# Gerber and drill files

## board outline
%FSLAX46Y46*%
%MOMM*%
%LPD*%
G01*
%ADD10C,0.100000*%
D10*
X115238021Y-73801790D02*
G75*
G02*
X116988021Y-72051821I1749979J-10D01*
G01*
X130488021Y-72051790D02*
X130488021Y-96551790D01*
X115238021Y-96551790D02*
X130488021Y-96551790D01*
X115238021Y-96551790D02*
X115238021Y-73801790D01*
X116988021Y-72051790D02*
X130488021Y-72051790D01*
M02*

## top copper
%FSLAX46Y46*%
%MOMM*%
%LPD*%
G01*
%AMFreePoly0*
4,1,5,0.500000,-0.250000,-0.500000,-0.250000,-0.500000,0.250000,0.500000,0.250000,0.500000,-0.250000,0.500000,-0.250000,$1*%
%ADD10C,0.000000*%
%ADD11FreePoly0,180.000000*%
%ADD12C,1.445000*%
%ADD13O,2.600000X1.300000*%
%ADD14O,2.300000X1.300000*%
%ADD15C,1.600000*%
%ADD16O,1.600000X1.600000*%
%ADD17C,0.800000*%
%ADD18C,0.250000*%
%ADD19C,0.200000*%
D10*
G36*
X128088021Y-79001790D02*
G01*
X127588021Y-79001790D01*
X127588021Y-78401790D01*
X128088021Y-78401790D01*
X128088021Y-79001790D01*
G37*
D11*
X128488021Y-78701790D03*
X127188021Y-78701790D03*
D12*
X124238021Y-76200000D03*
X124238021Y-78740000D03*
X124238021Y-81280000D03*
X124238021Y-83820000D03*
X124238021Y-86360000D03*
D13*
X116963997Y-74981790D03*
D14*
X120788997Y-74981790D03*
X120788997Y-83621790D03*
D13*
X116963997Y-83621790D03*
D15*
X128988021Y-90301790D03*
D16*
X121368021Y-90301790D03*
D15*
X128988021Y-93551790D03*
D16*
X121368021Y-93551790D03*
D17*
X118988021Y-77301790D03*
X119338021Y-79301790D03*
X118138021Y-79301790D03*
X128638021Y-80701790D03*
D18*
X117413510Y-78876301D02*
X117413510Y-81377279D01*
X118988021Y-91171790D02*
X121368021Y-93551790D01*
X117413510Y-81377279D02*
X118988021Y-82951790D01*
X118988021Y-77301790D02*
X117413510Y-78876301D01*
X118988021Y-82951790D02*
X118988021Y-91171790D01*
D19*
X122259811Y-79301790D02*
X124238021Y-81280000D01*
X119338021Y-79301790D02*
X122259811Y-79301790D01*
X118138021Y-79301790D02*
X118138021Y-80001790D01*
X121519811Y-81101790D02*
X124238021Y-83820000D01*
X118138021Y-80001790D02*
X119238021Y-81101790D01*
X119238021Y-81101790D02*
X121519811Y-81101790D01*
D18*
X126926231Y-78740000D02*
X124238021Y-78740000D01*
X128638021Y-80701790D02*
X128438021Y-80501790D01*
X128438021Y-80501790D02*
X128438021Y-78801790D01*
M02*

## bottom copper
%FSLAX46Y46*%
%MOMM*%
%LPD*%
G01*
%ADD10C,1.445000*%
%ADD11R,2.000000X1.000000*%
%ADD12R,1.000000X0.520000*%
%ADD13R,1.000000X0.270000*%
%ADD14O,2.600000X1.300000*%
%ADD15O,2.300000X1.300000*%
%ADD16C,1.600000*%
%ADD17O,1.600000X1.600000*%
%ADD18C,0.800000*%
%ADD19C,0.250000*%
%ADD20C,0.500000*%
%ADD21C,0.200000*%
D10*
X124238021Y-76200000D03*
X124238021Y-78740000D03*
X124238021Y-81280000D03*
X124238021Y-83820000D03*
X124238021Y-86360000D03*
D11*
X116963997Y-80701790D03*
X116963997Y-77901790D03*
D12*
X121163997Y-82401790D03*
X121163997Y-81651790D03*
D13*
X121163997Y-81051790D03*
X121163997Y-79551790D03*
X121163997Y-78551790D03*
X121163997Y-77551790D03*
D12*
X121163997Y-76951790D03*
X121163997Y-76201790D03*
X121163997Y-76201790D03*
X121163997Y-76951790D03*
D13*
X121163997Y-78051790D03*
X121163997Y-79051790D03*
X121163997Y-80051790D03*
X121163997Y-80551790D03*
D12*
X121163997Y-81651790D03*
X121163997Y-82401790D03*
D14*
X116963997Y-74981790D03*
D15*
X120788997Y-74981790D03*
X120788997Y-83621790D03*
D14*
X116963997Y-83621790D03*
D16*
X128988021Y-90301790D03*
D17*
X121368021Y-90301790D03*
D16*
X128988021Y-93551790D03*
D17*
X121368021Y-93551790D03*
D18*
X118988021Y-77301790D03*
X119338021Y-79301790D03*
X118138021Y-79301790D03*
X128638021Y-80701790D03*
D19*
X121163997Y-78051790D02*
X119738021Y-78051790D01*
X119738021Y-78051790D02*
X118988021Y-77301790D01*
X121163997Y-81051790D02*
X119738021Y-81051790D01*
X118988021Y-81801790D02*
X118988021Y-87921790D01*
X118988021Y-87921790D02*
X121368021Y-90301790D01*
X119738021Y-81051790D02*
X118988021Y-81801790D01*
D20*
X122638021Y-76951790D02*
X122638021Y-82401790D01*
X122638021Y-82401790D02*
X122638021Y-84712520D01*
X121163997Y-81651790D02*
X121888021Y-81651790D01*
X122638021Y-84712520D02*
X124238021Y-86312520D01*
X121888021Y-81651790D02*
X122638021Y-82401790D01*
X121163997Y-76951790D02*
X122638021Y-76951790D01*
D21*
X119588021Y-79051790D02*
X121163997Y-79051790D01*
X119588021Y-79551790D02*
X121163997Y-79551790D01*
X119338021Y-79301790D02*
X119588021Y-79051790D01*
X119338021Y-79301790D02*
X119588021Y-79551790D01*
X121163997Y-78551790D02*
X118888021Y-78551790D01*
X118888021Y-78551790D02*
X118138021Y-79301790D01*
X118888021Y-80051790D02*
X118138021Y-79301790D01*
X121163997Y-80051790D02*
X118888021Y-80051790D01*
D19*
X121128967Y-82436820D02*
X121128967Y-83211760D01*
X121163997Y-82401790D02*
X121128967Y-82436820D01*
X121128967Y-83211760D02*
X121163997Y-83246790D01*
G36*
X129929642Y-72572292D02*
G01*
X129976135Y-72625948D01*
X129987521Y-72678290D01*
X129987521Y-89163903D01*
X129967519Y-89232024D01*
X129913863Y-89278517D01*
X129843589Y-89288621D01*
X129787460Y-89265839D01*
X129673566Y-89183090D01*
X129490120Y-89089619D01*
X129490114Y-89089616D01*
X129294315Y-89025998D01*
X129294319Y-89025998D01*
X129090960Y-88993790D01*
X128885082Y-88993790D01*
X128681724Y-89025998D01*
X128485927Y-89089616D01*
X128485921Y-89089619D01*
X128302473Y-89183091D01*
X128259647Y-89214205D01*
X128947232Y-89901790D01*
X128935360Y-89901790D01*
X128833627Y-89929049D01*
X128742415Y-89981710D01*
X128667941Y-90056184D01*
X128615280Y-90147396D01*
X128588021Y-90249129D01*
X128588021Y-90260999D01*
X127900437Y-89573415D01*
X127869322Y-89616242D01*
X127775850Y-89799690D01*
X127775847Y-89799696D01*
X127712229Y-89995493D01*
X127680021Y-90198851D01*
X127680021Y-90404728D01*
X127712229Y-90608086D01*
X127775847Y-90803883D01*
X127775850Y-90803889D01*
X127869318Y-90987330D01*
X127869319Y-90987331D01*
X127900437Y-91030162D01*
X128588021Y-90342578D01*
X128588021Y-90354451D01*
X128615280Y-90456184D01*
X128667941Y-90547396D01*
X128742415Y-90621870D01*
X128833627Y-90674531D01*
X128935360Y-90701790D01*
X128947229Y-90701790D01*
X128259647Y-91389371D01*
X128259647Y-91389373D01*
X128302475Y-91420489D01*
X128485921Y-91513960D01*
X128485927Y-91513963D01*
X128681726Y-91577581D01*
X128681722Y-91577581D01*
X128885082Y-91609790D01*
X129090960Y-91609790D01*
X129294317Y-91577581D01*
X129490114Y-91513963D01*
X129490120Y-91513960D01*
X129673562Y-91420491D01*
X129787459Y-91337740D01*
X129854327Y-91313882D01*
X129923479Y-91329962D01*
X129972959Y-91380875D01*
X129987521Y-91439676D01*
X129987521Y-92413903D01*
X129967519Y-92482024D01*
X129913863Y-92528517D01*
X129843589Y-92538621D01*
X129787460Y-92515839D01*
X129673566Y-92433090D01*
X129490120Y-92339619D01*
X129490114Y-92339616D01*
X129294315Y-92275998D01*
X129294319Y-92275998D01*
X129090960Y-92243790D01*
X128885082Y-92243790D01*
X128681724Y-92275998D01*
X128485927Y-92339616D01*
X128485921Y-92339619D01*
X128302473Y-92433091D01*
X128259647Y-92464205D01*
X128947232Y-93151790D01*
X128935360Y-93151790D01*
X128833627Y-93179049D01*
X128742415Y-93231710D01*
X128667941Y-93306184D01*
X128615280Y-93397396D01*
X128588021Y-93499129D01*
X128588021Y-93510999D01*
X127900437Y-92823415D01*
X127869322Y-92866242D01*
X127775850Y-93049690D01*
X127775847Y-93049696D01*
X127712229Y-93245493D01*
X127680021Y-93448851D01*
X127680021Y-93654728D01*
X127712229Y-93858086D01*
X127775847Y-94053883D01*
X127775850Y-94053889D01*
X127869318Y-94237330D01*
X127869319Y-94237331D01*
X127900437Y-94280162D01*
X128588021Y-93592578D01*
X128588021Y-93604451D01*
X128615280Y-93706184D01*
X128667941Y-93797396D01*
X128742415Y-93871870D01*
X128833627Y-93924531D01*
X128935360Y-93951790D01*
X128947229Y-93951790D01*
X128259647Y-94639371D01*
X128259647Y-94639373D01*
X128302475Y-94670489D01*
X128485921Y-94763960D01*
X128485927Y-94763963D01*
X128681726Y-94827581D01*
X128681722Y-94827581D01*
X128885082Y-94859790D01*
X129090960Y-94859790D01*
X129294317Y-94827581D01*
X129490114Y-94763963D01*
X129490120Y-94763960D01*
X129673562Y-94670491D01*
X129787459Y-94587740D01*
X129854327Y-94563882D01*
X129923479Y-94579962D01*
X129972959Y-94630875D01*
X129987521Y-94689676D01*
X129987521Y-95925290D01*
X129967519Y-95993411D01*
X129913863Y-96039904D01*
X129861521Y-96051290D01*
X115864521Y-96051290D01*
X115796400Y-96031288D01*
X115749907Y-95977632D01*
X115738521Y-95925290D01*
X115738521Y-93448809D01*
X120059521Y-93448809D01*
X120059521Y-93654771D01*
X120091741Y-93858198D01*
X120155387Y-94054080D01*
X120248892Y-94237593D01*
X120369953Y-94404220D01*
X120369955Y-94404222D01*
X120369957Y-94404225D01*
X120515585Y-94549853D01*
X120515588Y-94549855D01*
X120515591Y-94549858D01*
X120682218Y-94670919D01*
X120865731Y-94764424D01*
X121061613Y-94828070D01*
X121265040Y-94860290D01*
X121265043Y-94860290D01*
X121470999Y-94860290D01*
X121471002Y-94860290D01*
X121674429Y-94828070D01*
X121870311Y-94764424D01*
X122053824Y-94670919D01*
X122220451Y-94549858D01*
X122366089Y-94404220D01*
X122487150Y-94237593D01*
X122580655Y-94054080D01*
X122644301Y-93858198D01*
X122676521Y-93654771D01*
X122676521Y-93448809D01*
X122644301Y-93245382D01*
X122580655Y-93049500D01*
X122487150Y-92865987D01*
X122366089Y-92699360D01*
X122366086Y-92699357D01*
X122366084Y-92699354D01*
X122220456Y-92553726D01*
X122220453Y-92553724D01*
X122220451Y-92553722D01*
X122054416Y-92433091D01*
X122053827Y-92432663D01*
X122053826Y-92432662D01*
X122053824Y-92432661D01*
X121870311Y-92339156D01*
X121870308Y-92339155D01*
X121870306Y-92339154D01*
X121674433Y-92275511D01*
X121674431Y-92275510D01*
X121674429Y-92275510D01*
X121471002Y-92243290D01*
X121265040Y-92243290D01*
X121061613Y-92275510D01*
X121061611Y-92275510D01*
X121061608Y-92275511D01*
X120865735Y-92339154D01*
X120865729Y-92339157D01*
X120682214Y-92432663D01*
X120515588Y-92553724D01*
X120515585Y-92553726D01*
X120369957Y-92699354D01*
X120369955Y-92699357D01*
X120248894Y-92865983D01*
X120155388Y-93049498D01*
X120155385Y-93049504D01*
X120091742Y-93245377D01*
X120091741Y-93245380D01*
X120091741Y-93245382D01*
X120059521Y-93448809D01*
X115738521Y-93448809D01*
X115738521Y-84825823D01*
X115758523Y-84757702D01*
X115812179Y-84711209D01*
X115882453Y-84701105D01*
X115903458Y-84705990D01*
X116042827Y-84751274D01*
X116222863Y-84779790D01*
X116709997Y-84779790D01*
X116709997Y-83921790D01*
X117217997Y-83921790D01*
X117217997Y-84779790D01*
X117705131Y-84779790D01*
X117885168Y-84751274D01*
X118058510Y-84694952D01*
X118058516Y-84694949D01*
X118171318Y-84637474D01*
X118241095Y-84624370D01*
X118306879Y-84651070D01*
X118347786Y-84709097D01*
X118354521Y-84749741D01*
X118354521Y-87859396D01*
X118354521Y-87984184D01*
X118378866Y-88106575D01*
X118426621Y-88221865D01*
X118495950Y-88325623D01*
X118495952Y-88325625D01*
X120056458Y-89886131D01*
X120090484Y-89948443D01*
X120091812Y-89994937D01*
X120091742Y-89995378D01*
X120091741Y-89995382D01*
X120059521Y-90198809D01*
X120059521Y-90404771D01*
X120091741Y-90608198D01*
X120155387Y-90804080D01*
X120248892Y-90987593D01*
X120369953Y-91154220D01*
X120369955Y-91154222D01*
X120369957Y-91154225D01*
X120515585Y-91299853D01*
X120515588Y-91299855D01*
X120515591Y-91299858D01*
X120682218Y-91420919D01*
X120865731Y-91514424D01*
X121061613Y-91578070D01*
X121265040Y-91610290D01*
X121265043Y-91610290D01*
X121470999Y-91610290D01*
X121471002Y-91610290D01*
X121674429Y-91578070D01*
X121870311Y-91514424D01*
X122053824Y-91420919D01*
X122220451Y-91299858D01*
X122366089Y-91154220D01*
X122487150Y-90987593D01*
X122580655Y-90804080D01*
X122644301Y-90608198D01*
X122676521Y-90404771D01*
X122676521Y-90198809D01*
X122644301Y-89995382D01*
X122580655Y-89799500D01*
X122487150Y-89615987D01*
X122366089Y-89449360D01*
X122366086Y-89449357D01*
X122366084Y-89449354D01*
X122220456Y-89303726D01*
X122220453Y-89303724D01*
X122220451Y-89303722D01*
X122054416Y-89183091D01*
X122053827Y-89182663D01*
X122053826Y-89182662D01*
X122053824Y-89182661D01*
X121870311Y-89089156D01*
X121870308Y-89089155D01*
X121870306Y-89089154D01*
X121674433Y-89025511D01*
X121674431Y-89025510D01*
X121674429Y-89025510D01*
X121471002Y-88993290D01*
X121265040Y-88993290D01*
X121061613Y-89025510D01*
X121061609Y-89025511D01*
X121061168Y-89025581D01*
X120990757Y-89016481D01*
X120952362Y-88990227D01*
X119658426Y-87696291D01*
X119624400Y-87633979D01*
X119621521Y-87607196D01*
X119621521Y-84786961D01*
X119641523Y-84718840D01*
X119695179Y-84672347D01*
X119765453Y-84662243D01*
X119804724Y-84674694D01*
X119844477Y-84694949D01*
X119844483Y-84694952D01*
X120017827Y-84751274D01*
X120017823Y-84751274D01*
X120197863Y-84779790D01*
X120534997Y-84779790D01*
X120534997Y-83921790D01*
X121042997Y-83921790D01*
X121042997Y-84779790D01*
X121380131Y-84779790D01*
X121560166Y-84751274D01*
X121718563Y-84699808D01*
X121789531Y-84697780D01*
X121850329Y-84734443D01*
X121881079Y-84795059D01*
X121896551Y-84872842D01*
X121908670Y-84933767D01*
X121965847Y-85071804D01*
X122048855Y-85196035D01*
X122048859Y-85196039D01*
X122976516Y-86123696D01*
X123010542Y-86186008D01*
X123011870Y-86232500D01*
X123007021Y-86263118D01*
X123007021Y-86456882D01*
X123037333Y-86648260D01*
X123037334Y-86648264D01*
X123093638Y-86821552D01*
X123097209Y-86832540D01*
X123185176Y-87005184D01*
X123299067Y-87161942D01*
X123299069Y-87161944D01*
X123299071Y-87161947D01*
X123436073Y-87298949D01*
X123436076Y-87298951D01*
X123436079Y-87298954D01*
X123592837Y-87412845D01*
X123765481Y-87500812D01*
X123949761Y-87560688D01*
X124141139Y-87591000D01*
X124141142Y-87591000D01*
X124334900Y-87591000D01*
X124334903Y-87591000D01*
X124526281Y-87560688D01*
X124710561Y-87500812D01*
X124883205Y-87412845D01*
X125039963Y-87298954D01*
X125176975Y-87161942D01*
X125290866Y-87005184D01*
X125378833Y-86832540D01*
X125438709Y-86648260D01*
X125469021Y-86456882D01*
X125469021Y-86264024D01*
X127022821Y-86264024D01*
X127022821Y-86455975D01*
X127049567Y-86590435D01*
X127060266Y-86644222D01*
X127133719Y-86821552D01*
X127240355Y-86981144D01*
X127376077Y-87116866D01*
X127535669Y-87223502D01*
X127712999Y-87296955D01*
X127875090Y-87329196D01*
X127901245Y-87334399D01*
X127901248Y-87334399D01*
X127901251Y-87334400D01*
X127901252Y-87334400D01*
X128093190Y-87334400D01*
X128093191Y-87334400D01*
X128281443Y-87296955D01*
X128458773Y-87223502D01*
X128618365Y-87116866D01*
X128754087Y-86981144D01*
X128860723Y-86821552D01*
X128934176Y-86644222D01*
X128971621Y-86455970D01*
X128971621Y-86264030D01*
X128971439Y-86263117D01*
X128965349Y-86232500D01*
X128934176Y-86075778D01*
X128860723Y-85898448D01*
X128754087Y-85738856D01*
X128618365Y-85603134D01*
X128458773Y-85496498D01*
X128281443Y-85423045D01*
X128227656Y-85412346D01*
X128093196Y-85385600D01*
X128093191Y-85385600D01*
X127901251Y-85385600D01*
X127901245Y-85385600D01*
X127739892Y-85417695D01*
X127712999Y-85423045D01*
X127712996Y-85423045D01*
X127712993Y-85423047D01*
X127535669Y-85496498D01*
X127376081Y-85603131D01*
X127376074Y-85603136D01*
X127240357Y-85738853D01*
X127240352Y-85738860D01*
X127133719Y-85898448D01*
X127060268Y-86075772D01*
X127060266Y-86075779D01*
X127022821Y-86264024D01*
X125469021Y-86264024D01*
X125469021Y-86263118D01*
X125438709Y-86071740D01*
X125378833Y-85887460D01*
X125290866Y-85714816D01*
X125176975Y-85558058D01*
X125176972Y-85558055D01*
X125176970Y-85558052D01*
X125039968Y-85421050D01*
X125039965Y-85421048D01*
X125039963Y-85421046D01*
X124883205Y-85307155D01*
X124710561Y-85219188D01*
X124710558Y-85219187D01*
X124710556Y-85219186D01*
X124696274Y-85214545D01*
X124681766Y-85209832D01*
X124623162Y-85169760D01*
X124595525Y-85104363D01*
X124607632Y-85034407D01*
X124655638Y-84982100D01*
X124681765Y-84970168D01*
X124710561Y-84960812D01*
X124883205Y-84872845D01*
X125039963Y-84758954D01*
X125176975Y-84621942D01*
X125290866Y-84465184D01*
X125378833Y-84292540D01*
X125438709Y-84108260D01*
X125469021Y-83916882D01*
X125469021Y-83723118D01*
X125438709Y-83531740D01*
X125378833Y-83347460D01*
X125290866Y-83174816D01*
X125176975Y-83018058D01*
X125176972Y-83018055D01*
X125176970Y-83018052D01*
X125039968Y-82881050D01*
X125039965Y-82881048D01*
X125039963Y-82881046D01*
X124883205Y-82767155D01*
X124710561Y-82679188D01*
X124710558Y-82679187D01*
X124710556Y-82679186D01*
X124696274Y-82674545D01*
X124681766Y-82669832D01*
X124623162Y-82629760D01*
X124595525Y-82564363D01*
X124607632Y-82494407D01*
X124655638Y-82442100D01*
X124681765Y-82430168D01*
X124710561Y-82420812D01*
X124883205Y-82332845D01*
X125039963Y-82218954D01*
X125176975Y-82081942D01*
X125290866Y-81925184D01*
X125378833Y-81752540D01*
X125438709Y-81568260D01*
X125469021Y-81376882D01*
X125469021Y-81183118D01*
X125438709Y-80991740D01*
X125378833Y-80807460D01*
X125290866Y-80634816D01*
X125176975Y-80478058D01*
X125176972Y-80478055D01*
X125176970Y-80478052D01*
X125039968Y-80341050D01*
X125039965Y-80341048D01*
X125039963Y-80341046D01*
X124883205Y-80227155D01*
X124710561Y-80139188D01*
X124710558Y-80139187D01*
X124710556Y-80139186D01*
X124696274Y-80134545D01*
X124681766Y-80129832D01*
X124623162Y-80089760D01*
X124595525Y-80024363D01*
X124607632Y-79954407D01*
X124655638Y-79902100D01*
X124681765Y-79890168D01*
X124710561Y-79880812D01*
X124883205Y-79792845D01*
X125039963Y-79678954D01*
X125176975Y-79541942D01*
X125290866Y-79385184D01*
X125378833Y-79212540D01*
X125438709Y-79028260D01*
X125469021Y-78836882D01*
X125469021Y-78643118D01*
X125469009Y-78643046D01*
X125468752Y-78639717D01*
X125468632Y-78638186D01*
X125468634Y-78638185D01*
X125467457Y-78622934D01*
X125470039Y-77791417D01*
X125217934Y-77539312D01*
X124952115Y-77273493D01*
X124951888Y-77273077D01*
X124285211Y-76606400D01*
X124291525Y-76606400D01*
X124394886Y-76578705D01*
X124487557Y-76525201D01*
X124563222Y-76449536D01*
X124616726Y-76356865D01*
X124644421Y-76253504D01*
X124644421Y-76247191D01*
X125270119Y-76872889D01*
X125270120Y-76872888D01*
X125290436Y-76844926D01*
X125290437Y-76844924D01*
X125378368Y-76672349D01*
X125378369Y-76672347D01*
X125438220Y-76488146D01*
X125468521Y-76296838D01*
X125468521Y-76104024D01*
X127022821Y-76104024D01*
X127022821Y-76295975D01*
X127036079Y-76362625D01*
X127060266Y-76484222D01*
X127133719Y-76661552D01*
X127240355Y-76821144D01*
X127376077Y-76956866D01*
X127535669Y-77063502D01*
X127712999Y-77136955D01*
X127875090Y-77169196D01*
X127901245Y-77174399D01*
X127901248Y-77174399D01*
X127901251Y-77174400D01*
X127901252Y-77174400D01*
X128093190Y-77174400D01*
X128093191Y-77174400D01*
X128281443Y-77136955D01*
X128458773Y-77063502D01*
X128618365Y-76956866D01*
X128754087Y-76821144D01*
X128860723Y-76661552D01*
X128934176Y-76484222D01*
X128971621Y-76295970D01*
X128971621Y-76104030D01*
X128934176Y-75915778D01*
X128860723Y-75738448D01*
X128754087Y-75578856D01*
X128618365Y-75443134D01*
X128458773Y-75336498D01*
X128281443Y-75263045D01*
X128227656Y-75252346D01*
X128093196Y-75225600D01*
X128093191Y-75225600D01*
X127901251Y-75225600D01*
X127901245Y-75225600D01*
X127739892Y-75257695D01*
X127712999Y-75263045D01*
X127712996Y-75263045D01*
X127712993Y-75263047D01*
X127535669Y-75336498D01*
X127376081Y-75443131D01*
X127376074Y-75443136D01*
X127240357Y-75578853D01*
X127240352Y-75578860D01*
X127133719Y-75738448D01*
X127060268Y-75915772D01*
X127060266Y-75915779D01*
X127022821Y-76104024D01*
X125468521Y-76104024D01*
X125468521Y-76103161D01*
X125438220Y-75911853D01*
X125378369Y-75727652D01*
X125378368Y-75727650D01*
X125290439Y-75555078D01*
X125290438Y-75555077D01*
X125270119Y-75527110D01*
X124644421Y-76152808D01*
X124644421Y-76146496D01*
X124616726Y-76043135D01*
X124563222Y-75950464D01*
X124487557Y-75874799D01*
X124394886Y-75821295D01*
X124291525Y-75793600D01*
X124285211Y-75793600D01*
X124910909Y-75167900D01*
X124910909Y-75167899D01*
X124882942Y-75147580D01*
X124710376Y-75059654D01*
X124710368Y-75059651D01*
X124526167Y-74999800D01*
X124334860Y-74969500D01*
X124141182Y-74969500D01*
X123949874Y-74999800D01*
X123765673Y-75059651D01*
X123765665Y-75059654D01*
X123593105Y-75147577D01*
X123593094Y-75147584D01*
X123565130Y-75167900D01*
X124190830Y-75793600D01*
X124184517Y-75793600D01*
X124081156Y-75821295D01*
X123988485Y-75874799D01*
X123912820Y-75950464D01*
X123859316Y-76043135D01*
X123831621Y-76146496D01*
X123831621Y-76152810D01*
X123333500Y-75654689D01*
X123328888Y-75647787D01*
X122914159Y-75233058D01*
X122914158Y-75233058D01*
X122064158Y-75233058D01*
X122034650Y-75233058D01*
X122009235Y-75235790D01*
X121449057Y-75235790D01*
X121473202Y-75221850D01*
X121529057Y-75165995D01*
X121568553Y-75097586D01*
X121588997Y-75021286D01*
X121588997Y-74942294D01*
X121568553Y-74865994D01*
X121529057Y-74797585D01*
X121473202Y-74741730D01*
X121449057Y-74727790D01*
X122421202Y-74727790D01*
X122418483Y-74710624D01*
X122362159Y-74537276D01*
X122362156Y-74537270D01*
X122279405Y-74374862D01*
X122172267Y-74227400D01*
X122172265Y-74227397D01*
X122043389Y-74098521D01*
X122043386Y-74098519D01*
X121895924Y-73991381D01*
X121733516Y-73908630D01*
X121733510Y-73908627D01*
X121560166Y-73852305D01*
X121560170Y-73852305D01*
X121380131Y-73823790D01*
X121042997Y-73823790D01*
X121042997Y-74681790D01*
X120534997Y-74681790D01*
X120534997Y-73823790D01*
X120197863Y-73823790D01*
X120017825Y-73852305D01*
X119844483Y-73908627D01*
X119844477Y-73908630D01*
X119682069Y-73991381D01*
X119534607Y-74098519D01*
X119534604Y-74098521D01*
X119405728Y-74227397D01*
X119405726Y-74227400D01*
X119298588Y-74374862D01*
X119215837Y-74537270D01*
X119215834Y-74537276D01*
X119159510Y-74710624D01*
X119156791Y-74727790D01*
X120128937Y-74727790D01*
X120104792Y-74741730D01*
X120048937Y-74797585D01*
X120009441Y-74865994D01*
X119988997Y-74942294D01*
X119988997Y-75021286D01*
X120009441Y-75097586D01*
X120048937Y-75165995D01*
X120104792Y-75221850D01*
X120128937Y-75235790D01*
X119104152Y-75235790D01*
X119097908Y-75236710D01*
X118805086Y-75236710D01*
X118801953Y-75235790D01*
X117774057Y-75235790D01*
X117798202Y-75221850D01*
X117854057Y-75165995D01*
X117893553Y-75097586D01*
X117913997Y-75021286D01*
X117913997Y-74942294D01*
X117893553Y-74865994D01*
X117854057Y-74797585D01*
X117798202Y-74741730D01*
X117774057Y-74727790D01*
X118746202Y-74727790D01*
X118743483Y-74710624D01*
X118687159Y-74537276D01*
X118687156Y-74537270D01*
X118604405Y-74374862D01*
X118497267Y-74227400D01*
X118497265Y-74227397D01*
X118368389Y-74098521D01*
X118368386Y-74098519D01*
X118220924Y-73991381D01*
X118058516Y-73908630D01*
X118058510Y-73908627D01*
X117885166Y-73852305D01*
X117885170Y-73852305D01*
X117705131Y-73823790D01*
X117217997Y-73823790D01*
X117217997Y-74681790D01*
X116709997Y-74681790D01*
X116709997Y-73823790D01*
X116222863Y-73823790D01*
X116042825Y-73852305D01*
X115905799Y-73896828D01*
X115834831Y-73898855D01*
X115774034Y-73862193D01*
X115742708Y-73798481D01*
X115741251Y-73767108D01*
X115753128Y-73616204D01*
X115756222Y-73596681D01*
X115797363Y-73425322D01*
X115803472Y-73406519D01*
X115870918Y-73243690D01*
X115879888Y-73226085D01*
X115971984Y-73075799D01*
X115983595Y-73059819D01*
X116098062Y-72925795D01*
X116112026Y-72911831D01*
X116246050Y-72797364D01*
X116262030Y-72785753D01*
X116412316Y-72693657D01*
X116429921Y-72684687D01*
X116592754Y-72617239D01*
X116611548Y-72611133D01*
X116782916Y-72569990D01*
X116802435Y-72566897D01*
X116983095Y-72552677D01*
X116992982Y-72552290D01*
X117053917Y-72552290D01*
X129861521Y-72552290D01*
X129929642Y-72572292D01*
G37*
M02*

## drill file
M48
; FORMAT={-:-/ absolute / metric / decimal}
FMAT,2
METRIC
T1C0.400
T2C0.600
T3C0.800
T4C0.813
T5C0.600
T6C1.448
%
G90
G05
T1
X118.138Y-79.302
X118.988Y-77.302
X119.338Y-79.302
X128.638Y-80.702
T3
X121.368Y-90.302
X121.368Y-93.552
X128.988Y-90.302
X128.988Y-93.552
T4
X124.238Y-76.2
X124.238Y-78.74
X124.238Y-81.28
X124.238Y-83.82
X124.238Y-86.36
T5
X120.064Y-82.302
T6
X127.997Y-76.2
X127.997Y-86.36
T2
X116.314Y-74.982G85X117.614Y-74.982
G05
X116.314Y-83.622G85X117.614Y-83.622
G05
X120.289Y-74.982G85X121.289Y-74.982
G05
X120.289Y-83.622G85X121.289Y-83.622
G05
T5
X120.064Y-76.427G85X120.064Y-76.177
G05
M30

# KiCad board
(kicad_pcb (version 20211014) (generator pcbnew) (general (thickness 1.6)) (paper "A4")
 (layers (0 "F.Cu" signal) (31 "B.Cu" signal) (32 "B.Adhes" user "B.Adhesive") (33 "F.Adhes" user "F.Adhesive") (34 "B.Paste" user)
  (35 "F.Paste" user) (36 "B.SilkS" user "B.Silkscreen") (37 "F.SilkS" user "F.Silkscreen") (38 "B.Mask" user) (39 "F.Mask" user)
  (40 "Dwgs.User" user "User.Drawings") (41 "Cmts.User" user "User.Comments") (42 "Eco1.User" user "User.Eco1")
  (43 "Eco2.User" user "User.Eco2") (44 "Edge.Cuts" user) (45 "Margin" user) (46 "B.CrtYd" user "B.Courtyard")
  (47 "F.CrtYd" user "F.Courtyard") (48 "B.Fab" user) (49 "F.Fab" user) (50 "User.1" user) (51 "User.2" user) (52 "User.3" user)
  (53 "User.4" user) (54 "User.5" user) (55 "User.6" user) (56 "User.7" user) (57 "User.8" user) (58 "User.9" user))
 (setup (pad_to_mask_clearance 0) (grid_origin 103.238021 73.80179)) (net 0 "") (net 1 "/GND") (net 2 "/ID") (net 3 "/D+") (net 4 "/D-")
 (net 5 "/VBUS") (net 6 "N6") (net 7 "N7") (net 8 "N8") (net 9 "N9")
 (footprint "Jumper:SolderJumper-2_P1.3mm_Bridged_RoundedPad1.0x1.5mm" (layer "F.Cu") (at 127.838021 78.70179 180)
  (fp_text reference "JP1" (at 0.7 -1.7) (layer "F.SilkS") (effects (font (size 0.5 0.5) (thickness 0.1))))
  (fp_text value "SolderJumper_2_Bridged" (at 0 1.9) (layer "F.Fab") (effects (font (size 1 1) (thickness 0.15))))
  (fp_poly (pts (xy 0.25 -0.3) (xy -0.25 -0.3) (xy -0.25 0.3) (xy 0.25 0.3)) (layer "F.Cu") (width 0) (fill solid))
  (pad "1" smd custom (at -0.65 0 180) (size 1 0.5) (layers "F.Cu" "F.Mask") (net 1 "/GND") (zone_connect 2)
   (options (clearance outline) (anchor rect)) (primitives))
  (pad "2" smd custom (at 0.65 0 180) (size 1 0.5) (layers "F.Cu" "F.Mask") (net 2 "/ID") (zone_connect 2)
   (options (clearance outline) (anchor rect)) (primitives)))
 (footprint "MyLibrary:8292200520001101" (layer "F.Cu") (at 124.238021 76.2)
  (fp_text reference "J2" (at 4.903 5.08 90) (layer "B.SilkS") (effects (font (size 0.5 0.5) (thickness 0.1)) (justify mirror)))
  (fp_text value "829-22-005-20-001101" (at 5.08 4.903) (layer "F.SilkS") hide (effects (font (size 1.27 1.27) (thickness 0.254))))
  (pad "" np_thru_hole circle (at 3.7592 10.16 90) (size 1.4478 1.4478) (drill 1.4478) (layers F&B.Cu *.Mask))
  (pad "" np_thru_hole circle (at 3.7592 0 90) (size 1.4478 1.4478) (drill 1.4478) (layers F&B.Cu *.Mask))
  (pad "1" thru_hole circle (at 0 0 90) (size 1.445 1.445) (drill 0.8128) (layers *.Cu *.Mask) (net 1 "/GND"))
  (pad "2" thru_hole circle (at 0 2.54 90) (size 1.445 1.445) (drill 0.8128) (layers *.Cu *.Mask) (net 2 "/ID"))
  (pad "3" thru_hole circle (at 0 5.08 90) (size 1.445 1.445) (drill 0.8128) (layers *.Cu *.Mask) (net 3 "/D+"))
  (pad "4" thru_hole circle (at 0 7.62 90) (size 1.445 1.445) (drill 0.8128) (layers *.Cu *.Mask) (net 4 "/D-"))
  (pad "5" thru_hole circle (at 0 10.16 90) (size 1.445 1.445) (drill 0.8128) (layers *.Cu *.Mask) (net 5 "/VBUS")))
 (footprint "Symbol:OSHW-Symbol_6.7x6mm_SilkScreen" (layer "F.Cu") (at 118.488021 79.30179 90)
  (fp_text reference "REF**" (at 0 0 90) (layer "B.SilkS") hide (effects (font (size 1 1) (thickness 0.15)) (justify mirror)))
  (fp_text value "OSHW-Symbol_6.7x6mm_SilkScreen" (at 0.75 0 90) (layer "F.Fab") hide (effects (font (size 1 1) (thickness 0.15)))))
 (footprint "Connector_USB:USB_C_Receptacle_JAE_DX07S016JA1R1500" (layer "B.Cu") (at 118.113997 79.30179 90)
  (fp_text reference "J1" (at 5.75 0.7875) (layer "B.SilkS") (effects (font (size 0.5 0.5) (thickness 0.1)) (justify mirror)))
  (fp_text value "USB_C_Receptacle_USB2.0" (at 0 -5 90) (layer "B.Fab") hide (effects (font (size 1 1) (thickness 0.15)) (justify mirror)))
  (pad "" smd rect (at -1.4 -1.15 90) (size 1 2) (layers "B.Cu" "B.Paste" "B.Mask"))
  (pad "" np_thru_hole circle (at -3 1.95 90) (size 0.6 0.6) (drill 0.6) (layers F&B.Cu *.Mask))
  (pad "" np_thru_hole oval (at 3 1.95 90) (size 0.85 0.6) (drill oval 0.85 0.6) (layers F&B.Cu *.Mask))
  (pad "" smd rect (at 1.4 -1.15 90) (size 1 2) (layers "B.Cu" "B.Paste" "B.Mask"))
  (pad "A1" smd rect (at -3.1 3.05 90) (size 0.52 1) (layers "B.Cu" "B.Paste" "B.Mask") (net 1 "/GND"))
  (pad "A4" smd rect (at -2.35 3.05 90) (size 0.52 1) (layers "B.Cu" "B.Paste" "B.Mask") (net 5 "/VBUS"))
  (pad "A5" smd rect (at -1.75 3.05 90) (size 0.27 1) (layers "B.Cu" "B.Paste" "B.Mask") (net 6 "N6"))
  (pad "A6" smd rect (at -0.25 3.05 90) (size 0.27 1) (layers "B.Cu" "B.Paste" "B.Mask") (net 3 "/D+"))
  (pad "A7" smd rect (at 0.75 3.05 90) (size 0.27 1) (layers "B.Cu" "B.Paste" "B.Mask") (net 4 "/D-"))
  (pad "A8" smd rect (at 1.75 3.05 90) (size 0.27 1) (layers "B.Cu" "B.Paste" "B.Mask") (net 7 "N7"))
  (pad "A9" smd rect (at 2.35 3.05 90) (size 0.52 1) (layers "B.Cu" "B.Paste" "B.Mask") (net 5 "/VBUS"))
  (pad "A12" smd rect (at 3.1 3.05 90) (size 0.52 1) (layers "B.Cu" "B.Paste" "B.Mask") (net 1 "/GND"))
  (pad "B1" smd rect (at 3.1 3.05 90) (size 0.52 1) (layers "B.Cu" "B.Paste" "B.Mask") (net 1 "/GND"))
  (pad "B4" smd rect (at 2.35 3.05 90) (size 0.52 1) (layers "B.Cu" "B.Paste" "B.Mask") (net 5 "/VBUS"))
  (pad "B5" smd rect (at 1.25 3.05 90) (size 0.27 1) (layers "B.Cu" "B.Paste" "B.Mask") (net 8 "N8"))
  (pad "B6" smd rect (at 0.25 3.05 90) (size 0.27 1) (layers "B.Cu" "B.Paste" "B.Mask") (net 3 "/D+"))
  (pad "B7" smd rect (at -0.75 3.05 90) (size 0.27 1) (layers "B.Cu" "B.Paste" "B.Mask") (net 4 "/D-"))
  (pad "B8" smd rect (at -1.25 3.05 90) (size 0.27 1) (layers "B.Cu" "B.Paste" "B.Mask") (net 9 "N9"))
  (pad "B9" smd rect (at -2.35 3.05 90) (size 0.52 1) (layers "B.Cu" "B.Paste" "B.Mask") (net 5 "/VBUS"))
  (pad "B12" smd rect (at -3.1 3.05 90) (size 0.52 1) (layers "B.Cu" "B.Paste" "B.Mask") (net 1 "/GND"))
  (pad "S1" thru_hole oval (at 4.32 -1.15 90) (size 1.3 2.6) (drill oval 0.6 1.9) (layers *.Cu *.Mask) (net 1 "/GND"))
  (pad "S1" thru_hole oval (at 4.32 2.675 90) (size 1.3 2.3) (drill oval 0.6 1.6) (layers *.Cu *.Mask) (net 1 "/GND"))
  (pad "S1" thru_hole oval (at -4.32 2.675 90) (size 1.3 2.3) (drill oval 0.6 1.6) (layers *.Cu *.Mask) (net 1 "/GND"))
  (pad "S1" thru_hole oval (at -4.32 -1.15 90) (size 1.3 2.6) (drill oval 0.6 1.9) (layers *.Cu *.Mask) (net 1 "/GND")))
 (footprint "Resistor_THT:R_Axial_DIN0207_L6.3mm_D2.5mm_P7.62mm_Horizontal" (layer "B.Cu") (at 128.988021 90.30179 180)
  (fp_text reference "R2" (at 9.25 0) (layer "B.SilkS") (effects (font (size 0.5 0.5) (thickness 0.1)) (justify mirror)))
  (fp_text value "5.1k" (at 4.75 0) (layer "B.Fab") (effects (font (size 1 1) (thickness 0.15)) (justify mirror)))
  (pad "1" thru_hole circle (at 0 0 180) (size 1.6 1.6) (drill 0.8) (layers *.Cu *.Mask) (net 1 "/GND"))
  (pad "2" thru_hole oval (at 7.62 0 180) (size 1.6 1.6) (drill 0.8) (layers *.Cu *.Mask) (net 6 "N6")))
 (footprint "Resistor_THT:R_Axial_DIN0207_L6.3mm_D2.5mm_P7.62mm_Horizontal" (layer "B.Cu") (at 128.988021 93.55179 180)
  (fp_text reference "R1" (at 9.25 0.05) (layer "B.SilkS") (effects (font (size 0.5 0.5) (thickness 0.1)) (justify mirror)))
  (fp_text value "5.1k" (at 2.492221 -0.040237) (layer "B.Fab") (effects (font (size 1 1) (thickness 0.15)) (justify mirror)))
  (pad "1" thru_hole circle (at 0 0 180) (size 1.6 1.6) (drill 0.8) (layers *.Cu *.Mask) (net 1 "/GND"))
  (pad "2" thru_hole oval (at 7.62 0 180) (size 1.6 1.6) (drill 0.8) (layers *.Cu *.Mask) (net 8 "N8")))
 (gr_arc (start 115.238021 73.80179) (mid 115.750587 72.564359) (end 116.988021 72.05179) (layer "Edge.Cuts") (width 0.1))
 (gr_line (start 130.488021 72.05179) (end 130.488021 96.55179) (layer "Edge.Cuts") (width 0.1))
 (gr_line (start 115.238021 96.55179) (end 130.488021 96.55179) (layer "Edge.Cuts") (width 0.1))
 (gr_line (start 115.238021 96.55179) (end 115.238021 73.80179) (layer "Edge.Cuts") (width 0.1))
 (gr_line (start 116.988021 72.05179) (end 130.488021 72.05179) (layer "Edge.Cuts") (width 0.1))
 (segment (start 117.41351 78.876301) (end 117.41351 81.377279) (width 0.25) (layer "F.Cu") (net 8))
 (segment (start 118.988021 91.17179) (end 121.368021 93.55179) (width 0.25) (layer "F.Cu") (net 8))
 (segment (start 117.41351 81.377279) (end 118.988021 82.95179) (width 0.25) (layer "F.Cu") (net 8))
 (segment (start 118.988021 77.30179) (end 117.41351 78.876301) (width 0.25) (layer "F.Cu") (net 8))
 (segment (start 118.988021 82.95179) (end 118.988021 91.17179) (width 0.25) (layer "F.Cu") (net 8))
 (via (at 118.988021 77.30179) (size 0.8) (drill 0.4) (layers "F.Cu" "B.Cu") (free) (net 8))
 (segment (start 121.163997 78.05179) (end 119.738021 78.05179) (width 0.25) (layer "B.Cu") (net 8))
 (segment (start 119.738021 78.05179) (end 118.988021 77.30179) (width 0.25) (layer "B.Cu") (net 8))
 (segment (start 121.163997 81.05179) (end 119.738021 81.05179) (width 0.25) (layer "B.Cu") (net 6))
 (segment (start 118.988021 81.80179) (end 118.988021 87.92179) (width 0.25) (layer "B.Cu") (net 6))
 (segment (start 118.988021 87.92179) (end 121.368021 90.30179) (width 0.25) (layer "B.Cu") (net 6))
 (segment (start 119.738021 81.05179) (end 118.988021 81.80179) (width 0.25) (layer "B.Cu") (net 6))
 (segment (start 122.638021 76.95179) (end 122.638021 82.40179) (width 0.5) (layer "B.Cu") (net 5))
 (segment (start 122.638021 82.40179) (end 122.638021 84.71252) (width 0.5) (layer "B.Cu") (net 5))
 (segment (start 121.163997 81.65179) (end 121.888021 81.65179) (width 0.5) (layer "B.Cu") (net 5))
 (segment (start 122.638021 84.71252) (end 124.238021 86.31252) (width 0.5) (layer "B.Cu") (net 5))
 (segment (start 121.888021 81.65179) (end 122.638021 82.40179) (width 0.5) (layer "B.Cu") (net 5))
 (segment (start 121.163997 76.95179) (end 122.638021 76.95179) (width 0.5) (layer "B.Cu") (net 5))
 (segment (start 122.259811 79.30179) (end 124.238021 81.28) (width 0.2) (layer "F.Cu") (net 3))
 (segment (start 119.338021 79.30179) (end 122.259811 79.30179) (width 0.2) (layer "F.Cu") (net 3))
 (via (at 119.338021 79.30179) (size 0.8) (drill 0.4) (layers "F.Cu" "B.Cu") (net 3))
 (segment (start 119.588021 79.05179) (end 121.163997 79.05179) (width 0.2) (layer "B.Cu") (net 3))
 (segment (start 119.588021 79.55179) (end 121.163997 79.55179) (width 0.2) (layer "B.Cu") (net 3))
 (segment (start 119.338021 79.30179) (end 119.588021 79.05179) (width 0.2) (layer "B.Cu") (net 3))
 (segment (start 119.338021 79.30179) (end 119.588021 79.55179) (width 0.2) (layer "B.Cu") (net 3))
 (segment (start 118.138021 79.30179) (end 118.138021 80.00179) (width 0.2) (layer "F.Cu") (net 4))
 (segment (start 121.519811 81.10179) (end 124.238021 83.82) (width 0.2) (layer "F.Cu") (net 4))
 (segment (start 118.138021 80.00179) (end 119.238021 81.10179) (width 0.2) (layer "F.Cu") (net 4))
 (segment (start 119.238021 81.10179) (end 121.519811 81.10179) (width 0.2) (layer "F.Cu") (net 4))
 (via (at 118.138021 79.30179) (size 0.8) (drill 0.4) (layers "F.Cu" "B.Cu") (free) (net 4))
 (segment (start 121.163997 78.55179) (end 118.888021 78.55179) (width 0.2) (layer "B.Cu") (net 4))
 (segment (start 118.888021 78.55179) (end 118.138021 79.30179) (width 0.2) (layer "B.Cu") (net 4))
 (segment (start 118.888021 80.05179) (end 118.138021 79.30179) (width 0.2) (layer "B.Cu") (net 4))
 (segment (start 121.163997 80.05179) (end 118.888021 80.05179) (width 0.2) (layer "B.Cu") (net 4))
 (segment (start 126.926231 78.74) (end 124.238021 78.74) (width 0.25) (layer "F.Cu") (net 2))
 (segment (start 128.638021 80.70179) (end 128.438021 80.50179) (width 0.25) (layer "F.Cu") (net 1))
 (segment (start 128.438021 80.50179) (end 128.438021 78.80179) (width 0.25) (layer "F.Cu") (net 1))
 (via (at 128.638021 80.70179) (size 0.8) (drill 0.4) (layers "F.Cu" "B.Cu") (free) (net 1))
 (segment (start 121.128967 82.43682) (end 121.128967 83.21176) (width 0.25) (layer "B.Cu") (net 1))
 (segment (start 121.163997 82.40179) (end 121.128967 82.43682) (width 0.25) (layer "B.Cu") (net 1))
 (segment (start 121.128967 83.21176) (end 121.163997 83.24679) (width 0.25) (layer "B.Cu") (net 1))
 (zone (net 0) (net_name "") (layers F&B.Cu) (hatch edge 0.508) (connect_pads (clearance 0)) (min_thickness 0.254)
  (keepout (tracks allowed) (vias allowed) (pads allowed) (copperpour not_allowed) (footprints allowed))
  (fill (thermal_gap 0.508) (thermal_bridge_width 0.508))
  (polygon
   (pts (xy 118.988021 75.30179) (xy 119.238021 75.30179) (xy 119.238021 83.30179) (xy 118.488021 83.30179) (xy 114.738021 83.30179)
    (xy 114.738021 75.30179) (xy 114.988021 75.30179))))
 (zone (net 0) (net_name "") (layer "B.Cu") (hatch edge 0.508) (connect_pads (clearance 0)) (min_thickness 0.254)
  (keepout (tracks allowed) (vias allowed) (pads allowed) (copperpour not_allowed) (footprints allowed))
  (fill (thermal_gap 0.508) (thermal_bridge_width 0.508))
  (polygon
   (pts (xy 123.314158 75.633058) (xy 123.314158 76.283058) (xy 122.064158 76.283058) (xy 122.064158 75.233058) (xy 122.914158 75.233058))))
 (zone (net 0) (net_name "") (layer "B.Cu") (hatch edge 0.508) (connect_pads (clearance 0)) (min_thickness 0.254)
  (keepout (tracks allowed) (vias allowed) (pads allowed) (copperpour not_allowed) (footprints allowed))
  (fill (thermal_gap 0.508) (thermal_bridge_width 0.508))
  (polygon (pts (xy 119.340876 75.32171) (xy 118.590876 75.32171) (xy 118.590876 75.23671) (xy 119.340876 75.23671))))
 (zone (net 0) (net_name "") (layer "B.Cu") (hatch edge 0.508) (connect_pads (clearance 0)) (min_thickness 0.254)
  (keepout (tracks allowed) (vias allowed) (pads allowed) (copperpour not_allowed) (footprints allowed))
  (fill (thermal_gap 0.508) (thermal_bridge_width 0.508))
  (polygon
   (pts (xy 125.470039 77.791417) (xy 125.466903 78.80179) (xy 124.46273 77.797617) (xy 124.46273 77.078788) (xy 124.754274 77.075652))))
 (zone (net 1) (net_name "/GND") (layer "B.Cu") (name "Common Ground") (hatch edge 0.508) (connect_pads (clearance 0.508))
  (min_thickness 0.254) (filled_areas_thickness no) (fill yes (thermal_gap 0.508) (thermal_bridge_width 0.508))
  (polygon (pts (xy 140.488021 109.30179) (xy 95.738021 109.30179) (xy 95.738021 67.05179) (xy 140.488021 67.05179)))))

